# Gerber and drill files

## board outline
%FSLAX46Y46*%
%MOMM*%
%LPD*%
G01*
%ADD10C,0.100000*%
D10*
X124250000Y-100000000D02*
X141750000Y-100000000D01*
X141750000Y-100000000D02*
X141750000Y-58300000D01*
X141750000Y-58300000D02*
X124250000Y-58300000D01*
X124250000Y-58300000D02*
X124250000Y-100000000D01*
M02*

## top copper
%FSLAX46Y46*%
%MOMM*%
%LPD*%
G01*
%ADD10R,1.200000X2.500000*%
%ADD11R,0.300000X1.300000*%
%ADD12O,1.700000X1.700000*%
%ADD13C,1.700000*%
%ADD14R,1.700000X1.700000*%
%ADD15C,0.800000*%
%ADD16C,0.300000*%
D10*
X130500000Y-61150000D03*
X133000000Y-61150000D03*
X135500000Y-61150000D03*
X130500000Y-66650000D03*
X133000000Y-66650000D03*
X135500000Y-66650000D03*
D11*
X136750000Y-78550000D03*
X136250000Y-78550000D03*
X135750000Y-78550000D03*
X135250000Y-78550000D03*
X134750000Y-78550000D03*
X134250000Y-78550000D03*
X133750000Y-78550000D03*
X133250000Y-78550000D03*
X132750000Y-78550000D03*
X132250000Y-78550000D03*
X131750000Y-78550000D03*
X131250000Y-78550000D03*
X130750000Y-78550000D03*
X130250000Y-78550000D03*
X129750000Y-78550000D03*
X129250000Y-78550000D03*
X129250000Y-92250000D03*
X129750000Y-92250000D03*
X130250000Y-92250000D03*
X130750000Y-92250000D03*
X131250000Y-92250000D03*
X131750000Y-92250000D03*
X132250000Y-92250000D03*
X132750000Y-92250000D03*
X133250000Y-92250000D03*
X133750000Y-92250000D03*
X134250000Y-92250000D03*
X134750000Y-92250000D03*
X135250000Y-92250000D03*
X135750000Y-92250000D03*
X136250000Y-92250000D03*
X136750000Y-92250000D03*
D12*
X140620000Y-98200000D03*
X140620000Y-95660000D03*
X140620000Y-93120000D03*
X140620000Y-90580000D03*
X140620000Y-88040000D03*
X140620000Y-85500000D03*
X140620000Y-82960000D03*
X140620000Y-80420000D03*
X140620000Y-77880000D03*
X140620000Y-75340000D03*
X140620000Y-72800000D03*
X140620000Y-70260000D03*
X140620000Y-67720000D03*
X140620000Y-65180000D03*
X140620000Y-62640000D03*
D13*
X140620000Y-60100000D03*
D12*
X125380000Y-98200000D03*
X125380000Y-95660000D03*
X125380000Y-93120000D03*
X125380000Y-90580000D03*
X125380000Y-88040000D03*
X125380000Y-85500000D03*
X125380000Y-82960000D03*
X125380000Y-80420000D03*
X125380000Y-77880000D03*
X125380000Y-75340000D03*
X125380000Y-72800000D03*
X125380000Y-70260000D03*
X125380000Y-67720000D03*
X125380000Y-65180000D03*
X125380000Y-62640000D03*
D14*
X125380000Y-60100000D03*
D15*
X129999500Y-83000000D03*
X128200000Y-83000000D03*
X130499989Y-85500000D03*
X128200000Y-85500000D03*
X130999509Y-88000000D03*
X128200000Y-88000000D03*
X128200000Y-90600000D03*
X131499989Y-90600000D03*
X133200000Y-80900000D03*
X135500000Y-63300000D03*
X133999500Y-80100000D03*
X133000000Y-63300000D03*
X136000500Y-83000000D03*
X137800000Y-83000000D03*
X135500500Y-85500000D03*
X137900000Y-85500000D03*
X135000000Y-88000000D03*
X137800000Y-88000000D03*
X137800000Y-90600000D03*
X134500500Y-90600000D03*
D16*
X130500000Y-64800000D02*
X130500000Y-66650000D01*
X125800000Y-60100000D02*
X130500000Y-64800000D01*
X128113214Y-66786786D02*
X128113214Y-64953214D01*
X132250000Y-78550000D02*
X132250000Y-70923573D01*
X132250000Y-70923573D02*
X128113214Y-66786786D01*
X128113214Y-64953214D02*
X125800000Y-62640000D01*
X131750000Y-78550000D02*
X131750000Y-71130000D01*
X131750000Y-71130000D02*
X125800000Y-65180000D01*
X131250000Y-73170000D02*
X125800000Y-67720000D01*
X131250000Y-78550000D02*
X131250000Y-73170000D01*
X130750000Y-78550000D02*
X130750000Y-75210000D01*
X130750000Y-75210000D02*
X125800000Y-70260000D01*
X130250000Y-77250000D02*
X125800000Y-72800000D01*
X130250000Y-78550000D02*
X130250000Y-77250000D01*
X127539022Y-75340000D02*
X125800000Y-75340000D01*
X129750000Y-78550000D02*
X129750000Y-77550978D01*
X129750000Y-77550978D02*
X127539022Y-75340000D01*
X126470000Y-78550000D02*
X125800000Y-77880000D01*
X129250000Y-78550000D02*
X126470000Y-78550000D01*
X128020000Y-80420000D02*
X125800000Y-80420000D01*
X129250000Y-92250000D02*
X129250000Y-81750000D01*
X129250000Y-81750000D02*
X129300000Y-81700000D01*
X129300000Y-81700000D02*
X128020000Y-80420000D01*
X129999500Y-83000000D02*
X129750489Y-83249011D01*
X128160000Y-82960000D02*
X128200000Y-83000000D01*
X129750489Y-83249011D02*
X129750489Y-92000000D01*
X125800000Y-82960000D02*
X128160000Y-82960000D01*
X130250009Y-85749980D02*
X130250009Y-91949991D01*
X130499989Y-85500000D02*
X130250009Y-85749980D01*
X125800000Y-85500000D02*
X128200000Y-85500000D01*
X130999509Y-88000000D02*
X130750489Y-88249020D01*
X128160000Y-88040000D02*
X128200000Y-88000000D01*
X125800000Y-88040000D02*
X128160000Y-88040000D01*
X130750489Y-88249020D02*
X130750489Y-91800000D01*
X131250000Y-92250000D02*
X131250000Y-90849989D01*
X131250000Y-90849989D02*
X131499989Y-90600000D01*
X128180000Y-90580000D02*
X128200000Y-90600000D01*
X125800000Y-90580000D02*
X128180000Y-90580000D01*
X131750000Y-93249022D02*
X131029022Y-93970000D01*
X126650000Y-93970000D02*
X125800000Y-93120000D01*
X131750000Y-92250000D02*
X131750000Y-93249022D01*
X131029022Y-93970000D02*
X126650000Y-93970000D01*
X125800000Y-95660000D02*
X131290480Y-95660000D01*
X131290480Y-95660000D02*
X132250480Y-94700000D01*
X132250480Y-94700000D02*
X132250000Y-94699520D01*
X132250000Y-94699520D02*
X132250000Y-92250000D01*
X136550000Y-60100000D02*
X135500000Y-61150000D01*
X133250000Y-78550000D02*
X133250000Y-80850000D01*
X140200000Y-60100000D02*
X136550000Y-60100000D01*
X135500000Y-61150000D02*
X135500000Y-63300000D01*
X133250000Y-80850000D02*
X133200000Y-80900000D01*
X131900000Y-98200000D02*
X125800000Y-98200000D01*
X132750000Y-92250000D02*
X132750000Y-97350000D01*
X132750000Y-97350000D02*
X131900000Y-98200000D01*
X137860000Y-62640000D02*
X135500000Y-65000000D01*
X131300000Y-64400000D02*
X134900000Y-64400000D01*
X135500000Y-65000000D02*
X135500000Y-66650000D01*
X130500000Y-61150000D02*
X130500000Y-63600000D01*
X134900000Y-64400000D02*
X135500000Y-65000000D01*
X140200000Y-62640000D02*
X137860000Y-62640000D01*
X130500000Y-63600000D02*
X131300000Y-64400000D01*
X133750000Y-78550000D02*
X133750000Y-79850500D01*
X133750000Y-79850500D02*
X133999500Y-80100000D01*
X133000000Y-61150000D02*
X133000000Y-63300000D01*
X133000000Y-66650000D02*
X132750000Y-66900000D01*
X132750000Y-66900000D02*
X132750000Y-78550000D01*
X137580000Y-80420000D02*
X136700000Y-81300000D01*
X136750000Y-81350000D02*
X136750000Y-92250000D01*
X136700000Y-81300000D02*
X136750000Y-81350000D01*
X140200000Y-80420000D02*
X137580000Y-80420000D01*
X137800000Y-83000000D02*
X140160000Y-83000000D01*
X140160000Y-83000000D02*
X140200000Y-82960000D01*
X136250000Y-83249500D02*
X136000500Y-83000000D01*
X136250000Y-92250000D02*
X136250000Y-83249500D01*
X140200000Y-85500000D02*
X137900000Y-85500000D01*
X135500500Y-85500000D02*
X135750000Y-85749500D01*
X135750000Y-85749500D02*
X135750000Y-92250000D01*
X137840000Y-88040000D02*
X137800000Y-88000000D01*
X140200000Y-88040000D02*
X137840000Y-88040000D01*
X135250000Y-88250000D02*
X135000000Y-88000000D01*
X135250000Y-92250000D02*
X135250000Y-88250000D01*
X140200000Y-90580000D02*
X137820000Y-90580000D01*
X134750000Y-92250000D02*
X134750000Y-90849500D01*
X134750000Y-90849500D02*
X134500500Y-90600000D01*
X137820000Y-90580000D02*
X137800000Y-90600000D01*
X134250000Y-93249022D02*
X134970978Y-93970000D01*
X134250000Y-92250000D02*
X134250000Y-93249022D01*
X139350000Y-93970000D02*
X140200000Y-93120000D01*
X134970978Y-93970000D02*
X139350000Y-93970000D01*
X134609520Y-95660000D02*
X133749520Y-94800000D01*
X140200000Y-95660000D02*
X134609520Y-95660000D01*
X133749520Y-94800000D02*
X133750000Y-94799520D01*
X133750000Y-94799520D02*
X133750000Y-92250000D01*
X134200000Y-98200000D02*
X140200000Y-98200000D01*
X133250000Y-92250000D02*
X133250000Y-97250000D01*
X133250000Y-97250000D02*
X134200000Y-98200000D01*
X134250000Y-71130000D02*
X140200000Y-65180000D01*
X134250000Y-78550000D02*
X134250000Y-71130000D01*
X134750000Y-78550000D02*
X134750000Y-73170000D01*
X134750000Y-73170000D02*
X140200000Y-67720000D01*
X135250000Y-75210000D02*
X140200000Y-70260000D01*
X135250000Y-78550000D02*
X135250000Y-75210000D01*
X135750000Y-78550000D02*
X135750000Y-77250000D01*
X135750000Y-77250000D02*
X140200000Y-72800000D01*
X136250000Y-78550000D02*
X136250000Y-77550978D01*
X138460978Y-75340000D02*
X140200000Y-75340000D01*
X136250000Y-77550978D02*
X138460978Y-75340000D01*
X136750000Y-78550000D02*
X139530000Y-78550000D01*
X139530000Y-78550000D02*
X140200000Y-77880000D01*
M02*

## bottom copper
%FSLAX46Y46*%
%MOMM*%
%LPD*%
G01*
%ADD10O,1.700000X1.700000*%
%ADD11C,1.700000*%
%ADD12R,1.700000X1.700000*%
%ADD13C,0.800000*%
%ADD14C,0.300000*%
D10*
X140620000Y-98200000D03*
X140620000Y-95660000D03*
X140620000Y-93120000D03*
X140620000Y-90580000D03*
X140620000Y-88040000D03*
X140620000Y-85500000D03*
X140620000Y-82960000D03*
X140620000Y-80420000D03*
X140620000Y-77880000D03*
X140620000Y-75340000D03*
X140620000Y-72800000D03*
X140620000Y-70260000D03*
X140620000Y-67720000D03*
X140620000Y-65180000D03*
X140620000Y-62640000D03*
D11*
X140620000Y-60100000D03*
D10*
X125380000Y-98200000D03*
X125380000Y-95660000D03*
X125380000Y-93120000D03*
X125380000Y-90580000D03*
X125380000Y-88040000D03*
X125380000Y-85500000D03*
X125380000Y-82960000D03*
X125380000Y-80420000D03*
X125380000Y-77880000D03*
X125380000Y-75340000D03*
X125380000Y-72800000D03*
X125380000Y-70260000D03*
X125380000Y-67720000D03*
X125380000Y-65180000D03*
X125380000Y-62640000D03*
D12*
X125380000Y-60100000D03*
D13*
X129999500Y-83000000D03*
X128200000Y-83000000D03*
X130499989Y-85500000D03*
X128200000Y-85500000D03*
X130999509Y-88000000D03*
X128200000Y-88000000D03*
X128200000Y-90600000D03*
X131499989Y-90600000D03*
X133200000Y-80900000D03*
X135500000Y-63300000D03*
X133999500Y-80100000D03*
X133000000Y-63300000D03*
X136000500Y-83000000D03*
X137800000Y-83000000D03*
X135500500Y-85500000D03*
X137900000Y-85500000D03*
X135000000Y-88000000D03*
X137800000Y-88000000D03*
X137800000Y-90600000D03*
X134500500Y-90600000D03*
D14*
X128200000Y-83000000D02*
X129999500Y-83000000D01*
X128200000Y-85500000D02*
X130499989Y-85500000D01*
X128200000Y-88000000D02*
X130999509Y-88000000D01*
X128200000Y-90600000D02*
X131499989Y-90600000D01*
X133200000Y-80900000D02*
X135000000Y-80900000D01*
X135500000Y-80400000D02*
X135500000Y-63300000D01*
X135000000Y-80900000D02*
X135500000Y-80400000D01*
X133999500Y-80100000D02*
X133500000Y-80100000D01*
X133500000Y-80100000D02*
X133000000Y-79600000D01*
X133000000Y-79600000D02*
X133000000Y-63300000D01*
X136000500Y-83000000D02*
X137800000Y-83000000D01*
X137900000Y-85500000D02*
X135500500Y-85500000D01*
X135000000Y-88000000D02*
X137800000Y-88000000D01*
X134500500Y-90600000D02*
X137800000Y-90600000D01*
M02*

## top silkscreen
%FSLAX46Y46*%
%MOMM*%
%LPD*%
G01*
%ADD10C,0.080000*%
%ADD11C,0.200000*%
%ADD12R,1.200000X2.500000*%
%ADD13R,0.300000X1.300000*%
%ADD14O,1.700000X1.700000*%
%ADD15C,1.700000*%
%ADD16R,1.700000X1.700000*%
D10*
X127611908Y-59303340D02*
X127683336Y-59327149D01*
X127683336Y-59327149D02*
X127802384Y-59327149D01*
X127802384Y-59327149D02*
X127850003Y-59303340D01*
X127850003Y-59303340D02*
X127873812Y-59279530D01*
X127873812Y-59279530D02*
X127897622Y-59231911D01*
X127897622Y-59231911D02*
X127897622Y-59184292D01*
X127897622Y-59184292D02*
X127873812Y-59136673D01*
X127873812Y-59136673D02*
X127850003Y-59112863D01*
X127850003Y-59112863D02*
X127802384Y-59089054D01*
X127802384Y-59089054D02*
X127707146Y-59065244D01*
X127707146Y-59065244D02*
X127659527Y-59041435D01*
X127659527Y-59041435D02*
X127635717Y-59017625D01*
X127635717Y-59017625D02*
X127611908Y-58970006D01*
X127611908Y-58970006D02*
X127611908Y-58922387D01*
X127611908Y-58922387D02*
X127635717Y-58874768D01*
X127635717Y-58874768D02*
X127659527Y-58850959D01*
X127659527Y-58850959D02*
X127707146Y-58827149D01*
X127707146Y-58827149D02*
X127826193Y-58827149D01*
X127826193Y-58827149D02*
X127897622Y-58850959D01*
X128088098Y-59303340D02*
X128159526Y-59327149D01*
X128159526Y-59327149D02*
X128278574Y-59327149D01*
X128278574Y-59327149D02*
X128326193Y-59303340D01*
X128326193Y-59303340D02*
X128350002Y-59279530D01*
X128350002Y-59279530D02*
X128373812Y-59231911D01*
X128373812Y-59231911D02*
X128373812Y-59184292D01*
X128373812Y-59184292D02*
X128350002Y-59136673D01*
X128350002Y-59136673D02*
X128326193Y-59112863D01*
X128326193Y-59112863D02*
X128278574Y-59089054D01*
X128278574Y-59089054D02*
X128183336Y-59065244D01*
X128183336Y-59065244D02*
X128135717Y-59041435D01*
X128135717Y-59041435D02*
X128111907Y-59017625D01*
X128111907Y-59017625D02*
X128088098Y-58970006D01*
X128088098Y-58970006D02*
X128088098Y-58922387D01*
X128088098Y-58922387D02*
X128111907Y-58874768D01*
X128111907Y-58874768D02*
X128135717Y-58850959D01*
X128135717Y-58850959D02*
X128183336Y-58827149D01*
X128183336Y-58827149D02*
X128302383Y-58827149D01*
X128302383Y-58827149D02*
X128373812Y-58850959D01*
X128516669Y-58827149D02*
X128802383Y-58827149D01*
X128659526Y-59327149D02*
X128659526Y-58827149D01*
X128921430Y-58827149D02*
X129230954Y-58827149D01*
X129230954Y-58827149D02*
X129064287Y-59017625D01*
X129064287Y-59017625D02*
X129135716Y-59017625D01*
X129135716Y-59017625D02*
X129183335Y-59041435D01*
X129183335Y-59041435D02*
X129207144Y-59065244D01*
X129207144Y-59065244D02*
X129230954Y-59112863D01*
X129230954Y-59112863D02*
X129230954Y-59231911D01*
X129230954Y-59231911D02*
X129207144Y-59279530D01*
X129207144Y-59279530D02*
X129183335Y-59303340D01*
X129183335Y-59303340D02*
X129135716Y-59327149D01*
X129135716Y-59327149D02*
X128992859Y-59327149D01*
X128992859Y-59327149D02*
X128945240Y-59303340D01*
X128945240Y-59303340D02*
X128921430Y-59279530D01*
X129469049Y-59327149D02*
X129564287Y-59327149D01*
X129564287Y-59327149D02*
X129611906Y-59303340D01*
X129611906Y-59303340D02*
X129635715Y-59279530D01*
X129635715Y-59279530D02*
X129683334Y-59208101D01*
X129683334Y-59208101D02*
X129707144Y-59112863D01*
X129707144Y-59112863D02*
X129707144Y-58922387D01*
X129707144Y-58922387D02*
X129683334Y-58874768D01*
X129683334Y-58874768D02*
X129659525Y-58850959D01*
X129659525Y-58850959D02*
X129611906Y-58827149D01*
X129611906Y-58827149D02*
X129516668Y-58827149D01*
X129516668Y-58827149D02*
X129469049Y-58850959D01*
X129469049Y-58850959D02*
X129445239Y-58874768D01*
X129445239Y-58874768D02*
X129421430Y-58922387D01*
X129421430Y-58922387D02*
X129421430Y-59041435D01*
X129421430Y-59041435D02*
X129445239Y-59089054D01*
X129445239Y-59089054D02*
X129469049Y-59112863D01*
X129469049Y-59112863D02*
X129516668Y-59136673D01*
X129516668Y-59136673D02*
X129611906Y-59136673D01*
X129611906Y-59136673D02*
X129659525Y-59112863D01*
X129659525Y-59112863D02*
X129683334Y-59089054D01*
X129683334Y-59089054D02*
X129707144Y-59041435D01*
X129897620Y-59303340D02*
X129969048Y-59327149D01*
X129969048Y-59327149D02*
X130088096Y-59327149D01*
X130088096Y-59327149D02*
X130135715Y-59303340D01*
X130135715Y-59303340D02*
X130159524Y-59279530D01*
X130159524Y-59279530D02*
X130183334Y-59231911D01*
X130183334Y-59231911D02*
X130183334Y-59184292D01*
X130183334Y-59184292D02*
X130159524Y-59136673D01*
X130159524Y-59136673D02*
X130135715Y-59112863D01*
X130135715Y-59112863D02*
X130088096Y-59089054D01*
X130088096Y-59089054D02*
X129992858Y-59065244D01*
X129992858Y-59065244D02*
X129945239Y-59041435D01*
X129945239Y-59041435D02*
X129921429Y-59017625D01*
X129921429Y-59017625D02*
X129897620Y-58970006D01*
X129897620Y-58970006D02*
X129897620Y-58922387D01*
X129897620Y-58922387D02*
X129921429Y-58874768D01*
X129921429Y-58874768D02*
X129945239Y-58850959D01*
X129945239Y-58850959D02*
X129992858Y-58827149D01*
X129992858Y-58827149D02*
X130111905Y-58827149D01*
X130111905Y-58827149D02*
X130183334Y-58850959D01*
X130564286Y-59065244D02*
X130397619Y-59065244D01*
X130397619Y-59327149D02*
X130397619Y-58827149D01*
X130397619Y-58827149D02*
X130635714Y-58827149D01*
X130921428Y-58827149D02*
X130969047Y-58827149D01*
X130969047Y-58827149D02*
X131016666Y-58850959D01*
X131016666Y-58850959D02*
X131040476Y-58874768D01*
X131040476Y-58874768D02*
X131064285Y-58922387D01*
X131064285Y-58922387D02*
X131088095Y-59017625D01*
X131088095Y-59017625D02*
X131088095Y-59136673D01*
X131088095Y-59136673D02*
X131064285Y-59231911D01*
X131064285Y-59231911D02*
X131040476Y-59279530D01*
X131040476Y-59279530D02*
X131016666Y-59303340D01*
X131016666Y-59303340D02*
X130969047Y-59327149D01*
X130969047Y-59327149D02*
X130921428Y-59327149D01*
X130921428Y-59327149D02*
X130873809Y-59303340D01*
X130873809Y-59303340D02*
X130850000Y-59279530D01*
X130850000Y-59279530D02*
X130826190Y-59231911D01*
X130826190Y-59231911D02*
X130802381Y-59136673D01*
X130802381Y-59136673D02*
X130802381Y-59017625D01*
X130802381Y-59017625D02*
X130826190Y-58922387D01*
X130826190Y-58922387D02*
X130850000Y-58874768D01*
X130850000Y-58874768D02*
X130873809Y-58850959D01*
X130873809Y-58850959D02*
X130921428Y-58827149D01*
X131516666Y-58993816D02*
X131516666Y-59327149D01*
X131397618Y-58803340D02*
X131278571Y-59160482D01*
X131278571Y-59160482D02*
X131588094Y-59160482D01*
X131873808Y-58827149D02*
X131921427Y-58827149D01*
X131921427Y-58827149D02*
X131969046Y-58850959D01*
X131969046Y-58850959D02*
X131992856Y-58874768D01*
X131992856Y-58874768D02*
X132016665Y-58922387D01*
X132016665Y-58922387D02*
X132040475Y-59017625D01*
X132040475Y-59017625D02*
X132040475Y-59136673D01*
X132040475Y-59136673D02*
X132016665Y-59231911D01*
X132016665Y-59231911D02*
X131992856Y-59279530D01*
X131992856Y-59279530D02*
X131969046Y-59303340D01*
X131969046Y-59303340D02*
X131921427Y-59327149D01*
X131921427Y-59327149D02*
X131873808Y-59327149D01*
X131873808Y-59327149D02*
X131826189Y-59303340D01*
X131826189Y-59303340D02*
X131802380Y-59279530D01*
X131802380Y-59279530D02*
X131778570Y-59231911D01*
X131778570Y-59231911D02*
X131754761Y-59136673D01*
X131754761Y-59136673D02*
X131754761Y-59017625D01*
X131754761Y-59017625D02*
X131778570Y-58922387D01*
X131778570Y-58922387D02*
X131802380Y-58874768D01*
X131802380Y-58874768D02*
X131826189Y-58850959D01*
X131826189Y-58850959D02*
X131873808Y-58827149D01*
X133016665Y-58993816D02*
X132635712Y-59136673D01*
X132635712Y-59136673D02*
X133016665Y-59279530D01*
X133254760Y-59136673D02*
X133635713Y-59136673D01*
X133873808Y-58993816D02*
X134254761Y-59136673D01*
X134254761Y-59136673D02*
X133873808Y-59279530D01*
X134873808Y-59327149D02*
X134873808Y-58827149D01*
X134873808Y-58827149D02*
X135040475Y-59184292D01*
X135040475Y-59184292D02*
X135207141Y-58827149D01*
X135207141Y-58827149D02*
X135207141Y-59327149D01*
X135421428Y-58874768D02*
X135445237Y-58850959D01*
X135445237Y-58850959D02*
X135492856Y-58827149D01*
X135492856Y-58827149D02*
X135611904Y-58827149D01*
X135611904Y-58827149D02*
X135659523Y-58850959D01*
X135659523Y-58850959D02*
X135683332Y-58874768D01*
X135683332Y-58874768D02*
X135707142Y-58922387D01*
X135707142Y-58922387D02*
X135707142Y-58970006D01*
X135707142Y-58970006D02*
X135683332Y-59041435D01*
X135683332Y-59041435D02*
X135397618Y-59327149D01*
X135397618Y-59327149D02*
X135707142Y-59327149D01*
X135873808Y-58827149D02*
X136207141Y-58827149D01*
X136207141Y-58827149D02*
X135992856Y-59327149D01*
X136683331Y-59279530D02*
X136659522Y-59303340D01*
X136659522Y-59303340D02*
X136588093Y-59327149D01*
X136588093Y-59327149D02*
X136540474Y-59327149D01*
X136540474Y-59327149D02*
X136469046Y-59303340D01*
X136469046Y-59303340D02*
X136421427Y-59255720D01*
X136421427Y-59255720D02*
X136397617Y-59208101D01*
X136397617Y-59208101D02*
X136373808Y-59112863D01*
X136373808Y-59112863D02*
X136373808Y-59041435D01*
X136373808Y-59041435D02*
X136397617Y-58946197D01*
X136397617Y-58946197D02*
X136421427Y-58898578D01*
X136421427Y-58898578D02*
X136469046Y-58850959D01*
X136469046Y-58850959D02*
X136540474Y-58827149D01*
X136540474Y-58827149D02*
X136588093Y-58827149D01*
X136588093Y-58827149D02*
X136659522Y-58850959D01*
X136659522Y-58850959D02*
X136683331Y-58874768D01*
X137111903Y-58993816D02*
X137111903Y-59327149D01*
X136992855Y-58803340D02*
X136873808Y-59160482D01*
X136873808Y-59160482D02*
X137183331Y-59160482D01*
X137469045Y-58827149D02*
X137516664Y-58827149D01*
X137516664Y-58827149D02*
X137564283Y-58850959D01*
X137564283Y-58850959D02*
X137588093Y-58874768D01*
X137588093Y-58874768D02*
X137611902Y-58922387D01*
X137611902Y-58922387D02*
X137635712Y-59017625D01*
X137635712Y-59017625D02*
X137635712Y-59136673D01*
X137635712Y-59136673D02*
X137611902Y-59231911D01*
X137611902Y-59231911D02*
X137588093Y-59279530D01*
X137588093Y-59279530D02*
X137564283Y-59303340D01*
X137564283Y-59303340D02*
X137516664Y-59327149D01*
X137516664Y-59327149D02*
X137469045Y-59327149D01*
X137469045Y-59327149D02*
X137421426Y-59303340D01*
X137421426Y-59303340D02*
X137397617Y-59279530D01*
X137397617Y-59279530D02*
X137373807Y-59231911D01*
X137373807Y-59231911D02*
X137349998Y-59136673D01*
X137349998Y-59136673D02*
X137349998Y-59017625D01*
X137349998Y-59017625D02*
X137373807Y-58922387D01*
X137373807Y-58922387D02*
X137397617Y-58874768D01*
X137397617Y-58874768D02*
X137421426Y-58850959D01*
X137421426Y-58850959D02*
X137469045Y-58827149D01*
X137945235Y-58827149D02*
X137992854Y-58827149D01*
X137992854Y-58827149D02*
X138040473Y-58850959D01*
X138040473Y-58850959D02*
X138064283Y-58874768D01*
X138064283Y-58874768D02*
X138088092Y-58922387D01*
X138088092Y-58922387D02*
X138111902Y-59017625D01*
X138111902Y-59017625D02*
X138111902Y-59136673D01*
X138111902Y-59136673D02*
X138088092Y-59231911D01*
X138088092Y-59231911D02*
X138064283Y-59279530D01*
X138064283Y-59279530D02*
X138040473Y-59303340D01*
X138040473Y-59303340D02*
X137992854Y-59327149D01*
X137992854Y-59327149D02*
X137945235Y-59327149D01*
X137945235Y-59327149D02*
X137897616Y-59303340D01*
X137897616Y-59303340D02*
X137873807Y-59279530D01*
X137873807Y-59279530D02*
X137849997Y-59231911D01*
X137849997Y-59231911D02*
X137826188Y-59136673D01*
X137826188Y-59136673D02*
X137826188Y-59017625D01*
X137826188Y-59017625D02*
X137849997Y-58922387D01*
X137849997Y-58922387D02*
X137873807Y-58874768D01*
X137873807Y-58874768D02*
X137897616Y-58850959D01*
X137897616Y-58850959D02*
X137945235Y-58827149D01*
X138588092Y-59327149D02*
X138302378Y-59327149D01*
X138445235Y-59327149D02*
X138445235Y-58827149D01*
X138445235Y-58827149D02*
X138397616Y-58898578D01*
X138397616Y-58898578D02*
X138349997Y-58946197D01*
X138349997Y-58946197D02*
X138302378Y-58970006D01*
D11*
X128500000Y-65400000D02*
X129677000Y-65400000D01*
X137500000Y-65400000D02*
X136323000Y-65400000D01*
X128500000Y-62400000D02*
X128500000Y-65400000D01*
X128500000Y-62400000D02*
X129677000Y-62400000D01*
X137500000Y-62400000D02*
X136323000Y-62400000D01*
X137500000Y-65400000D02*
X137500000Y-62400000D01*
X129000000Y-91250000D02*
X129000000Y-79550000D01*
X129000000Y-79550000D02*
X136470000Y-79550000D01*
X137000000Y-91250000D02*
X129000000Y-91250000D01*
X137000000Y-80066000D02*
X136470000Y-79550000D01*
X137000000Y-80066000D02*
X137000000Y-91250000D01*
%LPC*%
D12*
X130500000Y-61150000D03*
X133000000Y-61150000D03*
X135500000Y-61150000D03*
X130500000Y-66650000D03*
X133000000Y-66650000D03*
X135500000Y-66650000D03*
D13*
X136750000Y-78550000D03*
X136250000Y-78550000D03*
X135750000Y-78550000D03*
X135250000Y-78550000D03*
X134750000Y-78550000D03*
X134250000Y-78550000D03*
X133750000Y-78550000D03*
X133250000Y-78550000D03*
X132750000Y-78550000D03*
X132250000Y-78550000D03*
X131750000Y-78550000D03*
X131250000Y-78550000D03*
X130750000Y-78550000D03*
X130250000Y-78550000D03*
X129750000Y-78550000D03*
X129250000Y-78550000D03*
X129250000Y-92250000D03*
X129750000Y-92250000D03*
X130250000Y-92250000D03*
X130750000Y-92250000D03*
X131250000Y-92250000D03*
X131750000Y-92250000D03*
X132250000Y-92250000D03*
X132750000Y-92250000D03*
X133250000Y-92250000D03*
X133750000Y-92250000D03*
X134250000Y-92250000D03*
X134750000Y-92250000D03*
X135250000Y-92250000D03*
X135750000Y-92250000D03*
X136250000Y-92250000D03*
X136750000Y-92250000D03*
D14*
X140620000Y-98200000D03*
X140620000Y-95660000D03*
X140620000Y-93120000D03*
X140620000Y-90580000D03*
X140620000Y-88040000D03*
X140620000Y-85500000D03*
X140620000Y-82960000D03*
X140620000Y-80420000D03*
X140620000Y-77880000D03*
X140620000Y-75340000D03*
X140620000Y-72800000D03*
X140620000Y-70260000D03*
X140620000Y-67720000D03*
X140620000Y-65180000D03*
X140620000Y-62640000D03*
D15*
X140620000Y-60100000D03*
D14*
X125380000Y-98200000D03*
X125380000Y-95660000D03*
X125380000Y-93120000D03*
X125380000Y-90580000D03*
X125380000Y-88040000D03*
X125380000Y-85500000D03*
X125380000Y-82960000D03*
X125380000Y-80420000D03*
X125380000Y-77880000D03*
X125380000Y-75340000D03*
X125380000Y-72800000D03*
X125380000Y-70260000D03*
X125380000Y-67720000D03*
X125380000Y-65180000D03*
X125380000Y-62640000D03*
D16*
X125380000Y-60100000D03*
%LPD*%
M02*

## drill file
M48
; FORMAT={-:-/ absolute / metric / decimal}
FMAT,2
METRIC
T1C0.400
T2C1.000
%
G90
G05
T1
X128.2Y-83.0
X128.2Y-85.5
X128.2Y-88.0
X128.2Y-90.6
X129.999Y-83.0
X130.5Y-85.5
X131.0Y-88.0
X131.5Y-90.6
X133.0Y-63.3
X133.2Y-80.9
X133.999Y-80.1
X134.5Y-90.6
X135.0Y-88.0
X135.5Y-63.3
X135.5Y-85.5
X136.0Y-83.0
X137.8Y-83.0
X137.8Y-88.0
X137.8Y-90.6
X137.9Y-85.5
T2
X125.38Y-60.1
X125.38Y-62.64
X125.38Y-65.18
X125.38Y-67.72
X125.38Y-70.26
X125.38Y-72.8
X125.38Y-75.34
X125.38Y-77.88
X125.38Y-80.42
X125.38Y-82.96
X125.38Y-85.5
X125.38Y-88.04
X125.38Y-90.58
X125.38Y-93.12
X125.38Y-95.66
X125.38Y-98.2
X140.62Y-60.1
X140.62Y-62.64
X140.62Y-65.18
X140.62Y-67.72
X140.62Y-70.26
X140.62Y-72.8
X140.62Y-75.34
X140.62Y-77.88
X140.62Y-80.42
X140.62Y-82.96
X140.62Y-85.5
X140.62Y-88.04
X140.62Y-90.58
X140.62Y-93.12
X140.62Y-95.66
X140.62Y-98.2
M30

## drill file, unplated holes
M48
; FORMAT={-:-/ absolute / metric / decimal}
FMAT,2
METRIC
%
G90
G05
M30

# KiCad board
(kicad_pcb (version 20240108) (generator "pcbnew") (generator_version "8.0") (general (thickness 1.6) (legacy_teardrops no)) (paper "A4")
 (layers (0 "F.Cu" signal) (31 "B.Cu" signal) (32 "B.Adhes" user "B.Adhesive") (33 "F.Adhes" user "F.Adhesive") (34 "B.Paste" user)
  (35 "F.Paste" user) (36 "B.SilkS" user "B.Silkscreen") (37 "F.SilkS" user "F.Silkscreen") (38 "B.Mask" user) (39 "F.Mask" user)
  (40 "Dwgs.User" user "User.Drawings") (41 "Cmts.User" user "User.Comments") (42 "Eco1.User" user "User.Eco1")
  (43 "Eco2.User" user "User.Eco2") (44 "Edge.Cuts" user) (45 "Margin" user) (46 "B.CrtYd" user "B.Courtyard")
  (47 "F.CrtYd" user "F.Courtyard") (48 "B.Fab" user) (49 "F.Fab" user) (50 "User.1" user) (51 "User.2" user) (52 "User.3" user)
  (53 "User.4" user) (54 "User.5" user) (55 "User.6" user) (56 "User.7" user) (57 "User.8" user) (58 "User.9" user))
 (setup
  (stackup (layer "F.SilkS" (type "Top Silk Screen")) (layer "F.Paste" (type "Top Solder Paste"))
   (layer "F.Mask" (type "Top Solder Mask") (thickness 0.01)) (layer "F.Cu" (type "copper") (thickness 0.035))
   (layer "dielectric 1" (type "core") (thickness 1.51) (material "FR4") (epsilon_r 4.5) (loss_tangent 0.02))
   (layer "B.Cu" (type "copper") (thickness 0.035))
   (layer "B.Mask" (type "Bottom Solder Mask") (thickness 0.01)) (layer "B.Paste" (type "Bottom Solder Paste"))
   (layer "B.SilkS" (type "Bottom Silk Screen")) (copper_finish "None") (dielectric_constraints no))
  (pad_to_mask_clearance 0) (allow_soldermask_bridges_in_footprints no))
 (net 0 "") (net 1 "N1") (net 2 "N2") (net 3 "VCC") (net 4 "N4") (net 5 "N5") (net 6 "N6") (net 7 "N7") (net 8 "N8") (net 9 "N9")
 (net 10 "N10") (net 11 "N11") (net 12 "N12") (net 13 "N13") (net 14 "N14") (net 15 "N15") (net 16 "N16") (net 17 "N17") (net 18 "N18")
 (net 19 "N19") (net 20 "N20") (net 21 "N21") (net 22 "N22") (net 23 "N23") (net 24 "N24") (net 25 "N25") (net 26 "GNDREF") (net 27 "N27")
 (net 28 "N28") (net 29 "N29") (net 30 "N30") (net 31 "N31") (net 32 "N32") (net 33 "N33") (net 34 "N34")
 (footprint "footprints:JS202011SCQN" (layer "F.Cu") (at 133 63.9)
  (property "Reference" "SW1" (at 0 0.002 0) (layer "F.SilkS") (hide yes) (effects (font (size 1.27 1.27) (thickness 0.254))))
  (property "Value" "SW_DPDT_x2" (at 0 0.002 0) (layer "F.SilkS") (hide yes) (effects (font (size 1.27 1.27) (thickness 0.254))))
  (fp_line (start -4.5 -1.5) (end -4.5 1.5) (stroke (width 0.2) (type solid)) (layer "F.SilkS"))
  (fp_line (start -4.5 -1.5) (end -3.323 -1.5) (stroke (width 0.2) (type solid)) (layer "F.SilkS"))
  (fp_line (start -4.5 1.5) (end -3.323 1.5) (stroke (width 0.2) (type solid)) (layer "F.SilkS"))
  (fp_line (start 4.5 -1.5) (end 3.323 -1.5) (stroke (width 0.2) (type solid)) (layer "F.SilkS"))
  (fp_line (start 4.5 1.5) (end 3.323 1.5) (stroke (width 0.2) (type solid)) (layer "F.SilkS"))
  (fp_line (start 4.5 1.5) (end 4.5 -1.5) (stroke (width 0.2) (type solid)) (layer "F.SilkS"))
  (pad "1" smd rect (at -2.5 -2.75) (size 1.2 2.5) (layers "F.Cu" "F.Paste" "F.Mask") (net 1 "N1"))
  (pad "2" smd rect (at 0 -2.75) (size 1.2 2.5) (layers "F.Cu" "F.Paste" "F.Mask") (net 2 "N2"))
  (pad "3" smd rect (at 2.5 -2.75) (size 1.2 2.5) (layers "F.Cu" "F.Paste" "F.Mask") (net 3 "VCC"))
  (pad "4" smd rect (at -2.5 2.75) (size 1.2 2.5) (layers "F.Cu" "F.Paste" "F.Mask") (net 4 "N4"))
  (pad "5" smd rect (at 0 2.75) (size 1.2 2.5) (layers "F.Cu" "F.Paste" "F.Mask") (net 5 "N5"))
  (pad "6" smd rect (at 2.5 2.75) (size 1.2 2.5) (layers "F.Cu" "F.Paste" "F.Mask") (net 1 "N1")))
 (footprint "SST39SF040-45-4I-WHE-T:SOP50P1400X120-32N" (layer "F.Cu") (at 133 85.4 -90)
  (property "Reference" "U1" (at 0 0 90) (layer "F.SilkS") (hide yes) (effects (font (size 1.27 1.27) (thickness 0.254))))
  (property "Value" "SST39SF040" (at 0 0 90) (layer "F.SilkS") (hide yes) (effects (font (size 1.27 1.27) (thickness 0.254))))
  (fp_line (start -5.85 4) (end -5.85 -3.47) (stroke (width 0.2) (type solid)) (layer "F.SilkS"))
  (fp_line (start 5.85 4) (end -5.85 4) (stroke (width 0.2) (type solid)) (layer "F.SilkS"))
  (fp_line (start -5.334 -4) (end -5.85 -3.47) (stroke (width 0.2) (type solid)) (layer "F.SilkS"))
  (fp_line (start -5.334 -4) (end 5.85 -4) (stroke (width 0.2) (type solid)) (layer "F.SilkS"))
  (fp_line (start 5.85 -4) (end 5.85 4) (stroke (width 0.2) (type solid)) (layer "F.SilkS"))
  (pad "1" smd rect (at -6.85 -3.75) (size 0.3 1.3) (layers "F.Cu" "F.Paste" "F.Mask") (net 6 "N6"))
  (pad "2" smd rect (at -6.85 -3.25) (size 0.3 1.3) (layers "F.Cu" "F.Paste" "F.Mask") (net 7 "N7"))
  (pad "3" smd rect (at -6.85 -2.75) (size 0.3 1.3) (layers "F.Cu" "F.Paste" "F.Mask") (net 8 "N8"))
  (pad "4" smd rect (at -6.85 -2.25) (size 0.3 1.3) (layers "F.Cu" "F.Paste" "F.Mask") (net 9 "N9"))
  (pad "5" smd rect (at -6.85 -1.75) (size 0.3 1.3) (layers "F.Cu" "F.Paste" "F.Mask") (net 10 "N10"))
  (pad "6" smd rect (at -6.85 -1.25) (size 0.3 1.3) (layers "F.Cu" "F.Paste" "F.Mask") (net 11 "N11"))
  (pad "7" smd rect (at -6.85 -0.75) (size 0.3 1.3) (layers "F.Cu" "F.Paste" "F.Mask") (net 2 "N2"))
  (pad "8" smd rect (at -6.85 -0.25) (size 0.3 1.3) (layers "F.Cu" "F.Paste" "F.Mask") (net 3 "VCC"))
  (pad "9" smd rect (at -6.85 0.25) (size 0.3 1.3) (layers "F.Cu" "F.Paste" "F.Mask") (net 5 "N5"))
  (pad "10" smd rect (at -6.85 0.75) (size 0.3 1.3) (layers "F.Cu" "F.Paste" "F.Mask") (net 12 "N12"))
  (pad "11" smd rect (at -6.85 1.25) (size 0.3 1.3) (layers "F.Cu" "F.Paste" "F.Mask") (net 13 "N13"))
  (pad "12" smd rect (at -6.85 1.75) (size 0.3 1.3) (layers "F.Cu" "F.Paste" "F.Mask") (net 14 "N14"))
  (pad "13" smd rect (at -6.85 2.25) (size 0.3 1.3) (layers "F.Cu" "F.Paste" "F.Mask") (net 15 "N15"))
  (pad "14" smd rect (at -6.85 2.75) (size 0.3 1.3) (layers "F.Cu" "F.Paste" "F.Mask") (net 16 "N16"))
  (pad "15" smd rect (at -6.85 3.25) (size 0.3 1.3) (layers "F.Cu" "F.Paste" "F.Mask") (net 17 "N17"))
  (pad "16" smd rect (at -6.85 3.75) (size 0.3 1.3) (layers "F.Cu" "F.Paste" "F.Mask") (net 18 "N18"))
  (pad "17" smd rect (at 6.85 3.75) (size 0.3 1.3) (layers "F.Cu" "F.Paste" "F.Mask") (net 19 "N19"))
  (pad "18" smd rect (at 6.85 3.25) (size 0.3 1.3) (layers "F.Cu" "F.Paste" "F.Mask") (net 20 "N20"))
  (pad "19" smd rect (at 6.85 2.75) (size 0.3 1.3) (layers "F.Cu" "F.Paste" "F.Mask") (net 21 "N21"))
  (pad "20" smd rect (at 6.85 2.25) (size 0.3 1.3) (layers "F.Cu" "F.Paste" "F.Mask") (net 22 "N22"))
  (pad "21" smd rect (at 6.85 1.75) (size 0.3 1.3) (layers "F.Cu" "F.Paste" "F.Mask") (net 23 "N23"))
  (pad "22" smd rect (at 6.85 1.25) (size 0.3 1.3) (layers "F.Cu" "F.Paste" "F.Mask") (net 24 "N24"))
  (pad "23" smd rect (at 6.85 0.75) (size 0.3 1.3) (layers "F.Cu" "F.Paste" "F.Mask") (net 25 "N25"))
  (pad "24" smd rect (at 6.85 0.25) (size 0.3 1.3) (layers "F.Cu" "F.Paste" "F.Mask") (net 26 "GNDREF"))
  (pad "25" smd rect (at 6.85 -0.25) (size 0.3 1.3) (layers "F.Cu" "F.Paste" "F.Mask") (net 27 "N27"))
  (pad "26" smd rect (at 6.85 -0.75) (size 0.3 1.3) (layers "F.Cu" "F.Paste" "F.Mask") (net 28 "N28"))
  (pad "27" smd rect (at 6.85 -1.25) (size 0.3 1.3) (layers "F.Cu" "F.Paste" "F.Mask") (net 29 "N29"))
  (pad "28" smd rect (at 6.85 -1.75) (size 0.3 1.3) (layers "F.Cu" "F.Paste" "F.Mask") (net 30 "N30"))
  (pad "29" smd rect (at 6.85 -2.25) (size 0.3 1.3) (layers "F.Cu" "F.Paste" "F.Mask") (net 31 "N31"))
  (pad "30" smd rect (at 6.85 -2.75) (size 0.3 1.3) (layers "F.Cu" "F.Paste" "F.Mask") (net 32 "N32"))
  (pad "31" smd rect (at 6.85 -3.25) (size 0.3 1.3) (layers "F.Cu" "F.Paste" "F.Mask") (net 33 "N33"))
  (pad "32" smd rect (at 6.85 -3.75) (size 0.3 1.3) (layers "F.Cu" "F.Paste" "F.Mask") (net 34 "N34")))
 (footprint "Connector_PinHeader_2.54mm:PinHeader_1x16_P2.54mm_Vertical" (layer "F.Cu") (at 140.62 60.1)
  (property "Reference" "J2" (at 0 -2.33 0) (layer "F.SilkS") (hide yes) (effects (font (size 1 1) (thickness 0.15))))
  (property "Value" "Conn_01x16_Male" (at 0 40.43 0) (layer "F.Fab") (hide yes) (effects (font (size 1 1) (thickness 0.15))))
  (pad "17" thru_hole oval (at 0 38.1) (size 1.7 1.7) (drill 1) (layers "*.Cu" "*.Mask") (remove_unused_layers no) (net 27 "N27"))
  (pad "18" thru_hole oval (at 0 35.56) (size 1.7 1.7) (drill 1) (layers "*.Cu" "*.Mask") (remove_unused_layers no) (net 28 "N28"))
  (pad "19" thru_hole oval (at 0 33.02) (size 1.7 1.7) (drill 1) (layers "*.Cu" "*.Mask") (remove_unused_layers no) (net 29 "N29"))
  (pad "20" thru_hole oval (at 0 30.48) (size 1.7 1.7) (drill 1) (layers "*.Cu" "*.Mask") (remove_unused_layers no) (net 30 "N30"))
  (pad "21" thru_hole oval (at 0 27.94) (size 1.7 1.7) (drill 1) (layers "*.Cu" "*.Mask") (remove_unused_layers no) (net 31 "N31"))
  (pad "22" thru_hole oval (at 0 25.4) (size 1.7 1.7) (drill 1) (layers "*.Cu" "*.Mask") (remove_unused_layers no) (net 32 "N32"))
  (pad "23" thru_hole oval (at 0 22.86) (size 1.7 1.7) (drill 1) (layers "*.Cu" "*.Mask") (remove_unused_layers no) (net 33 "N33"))
  (pad "24" thru_hole oval (at 0 20.32) (size 1.7 1.7) (drill 1) (layers "*.Cu" "*.Mask") (remove_unused_layers no) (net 34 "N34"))
  (pad "25" thru_hole oval (at 0 17.78) (size 1.7 1.7) (drill 1) (layers "*.Cu" "*.Mask") (remove_unused_layers no) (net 6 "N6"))
  (pad "26" thru_hole oval (at 0 15.24) (size 1.7 1.7) (drill 1) (layers "*.Cu" "*.Mask") (remove_unused_layers no) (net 7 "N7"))
  (pad "27" thru_hole oval (at 0 12.7) (size 1.7 1.7) (drill 1) (layers "*.Cu" "*.Mask") (remove_unused_layers no) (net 8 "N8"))
  (pad "28" thru_hole oval (at 0 10.16) (size 1.7 1.7) (drill 1) (layers "*.Cu" "*.Mask") (remove_unused_layers no) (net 9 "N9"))
  (pad "29" thru_hole oval (at 0 7.62) (size 1.7 1.7) (drill 1) (layers "*.Cu" "*.Mask") (remove_unused_layers no) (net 10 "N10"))
  (pad "30" thru_hole oval (at 0 5.08) (size 1.7 1.7) (drill 1) (layers "*.Cu" "*.Mask") (remove_unused_layers no) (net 11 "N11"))
  (pad "31" thru_hole oval (at 0 2.54) (size 1.7 1.7) (drill 1) (layers "*.Cu" "*.Mask") (remove_unused_layers no) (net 1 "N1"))
  (pad "32" thru_hole circle (at 0 0) (size 1.7 1.7) (drill 1) (layers "*.Cu" "*.Mask") (remove_unused_layers no) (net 3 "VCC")))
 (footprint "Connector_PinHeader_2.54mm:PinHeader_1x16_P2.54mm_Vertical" (layer "F.Cu") (at 125.38 60.1)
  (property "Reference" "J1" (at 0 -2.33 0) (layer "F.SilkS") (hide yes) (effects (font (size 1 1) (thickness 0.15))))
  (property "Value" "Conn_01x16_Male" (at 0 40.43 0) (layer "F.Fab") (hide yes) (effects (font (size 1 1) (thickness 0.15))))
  (pad "1" thru_hole rect (at 0 0) (size 1.7 1.7) (drill 1) (layers "*.Cu" "*.Mask") (remove_unused_layers no) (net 4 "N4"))
  (pad "2" thru_hole oval (at 0 2.54) (size 1.7 1.7) (drill 1) (layers "*.Cu" "*.Mask") (remove_unused_layers no) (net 12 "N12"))
  (pad "3" thru_hole oval (at 0 5.08) (size 1.7 1.7) (drill 1) (layers "*.Cu" "*.Mask") (remove_unused_layers no) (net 13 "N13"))
  (pad "4" thru_hole oval (at 0 7.62) (size 1.7 1.7) (drill 1) (layers "*.Cu" "*.Mask") (remove_unused_layers no) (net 14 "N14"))
  (pad "5" thru_hole oval (at 0 10.16) (size 1.7 1.7) (drill 1) (layers "*.Cu" "*.Mask") (remove_unused_layers no) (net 15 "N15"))
  (pad "6" thru_hole oval (at 0 12.7) (size 1.7 1.7) (drill 1) (layers "*.Cu" "*.Mask") (remove_unused_layers no) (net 16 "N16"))
  (pad "7" thru_hole oval (at 0 15.24) (size 1.7 1.7) (drill 1) (layers "*.Cu" "*.Mask") (remove_unused_layers no) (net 17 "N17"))
  (pad "8" thru_hole oval (at 0 17.78) (size 1.7 1.7) (drill 1) (layers "*.Cu" "*.Mask") (remove_unused_layers no) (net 18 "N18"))
  (pad "9" thru_hole oval (at 0 20.32) (size 1.7 1.7) (drill 1) (layers "*.Cu" "*.Mask") (remove_unused_layers no) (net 19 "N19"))
  (pad "10" thru_hole oval (at 0 22.86) (size 1.7 1.7) (drill 1) (layers "*.Cu" "*.Mask") (remove_unused_layers no) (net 20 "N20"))
  (pad "11" thru_hole oval (at 0 25.4) (size 1.7 1.7) (drill 1) (layers "*.Cu" "*.Mask") (remove_unused_layers no) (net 21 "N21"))
  (pad "12" thru_hole oval (at 0 27.94) (size 1.7 1.7) (drill 1) (layers "*.Cu" "*.Mask") (remove_unused_layers no) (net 22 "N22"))
  (pad "13" thru_hole oval (at 0 30.48) (size 1.7 1.7) (drill 1) (layers "*.Cu" "*.Mask") (remove_unused_layers no) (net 23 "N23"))
  (pad "14" thru_hole oval (at 0 33.02) (size 1.7 1.7) (drill 1) (layers "*.Cu" "*.Mask") (remove_unused_layers no) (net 24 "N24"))
  (pad "15" thru_hole oval (at 0 35.56) (size 1.7 1.7) (drill 1) (layers "*.Cu" "*.Mask") (remove_unused_layers no) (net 25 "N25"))
  (pad "16" thru_hole oval (at 0 38.1) (size 1.7 1.7) (drill 1) (layers "*.Cu" "*.Mask") (remove_unused_layers no) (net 26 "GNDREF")))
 (gr_line (start 124.25 100) (end 141.75 100) (stroke (width 0.1) (type solid)) (layer "Edge.Cuts"))
 (gr_line (start 141.75 100) (end 141.75 58.3) (stroke (width 0.1) (type solid)) (layer "Edge.Cuts"))
 (gr_line (start 141.75 58.3) (end 124.25 58.3) (stroke (width 0.1) (type solid)) (layer "Edge.Cuts"))
 (gr_line (start 124.25 58.3) (end 124.25 100) (stroke (width 0.1) (type solid)) (layer "Edge.Cuts"))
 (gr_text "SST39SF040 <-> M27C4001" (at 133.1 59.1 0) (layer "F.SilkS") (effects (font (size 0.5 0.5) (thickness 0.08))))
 (segment (start 130.5 64.8) (end 130.5 66.65) (width 0.3) (layer "F.Cu") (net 4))
 (segment (start 125.8 60.1) (end 130.5 64.8) (width 0.3) (layer "F.Cu") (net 4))
 (segment (start 128.113214 66.786786) (end 128.113214 64.953214) (width 0.3) (layer "F.Cu") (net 12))
 (segment (start 132.25 78.55) (end 132.25 70.923573) (width 0.3) (layer "F.Cu") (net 12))
 (segment (start 132.25 70.923573) (end 128.113214 66.786786) (width 0.3) (layer "F.Cu") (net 12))
 (segment (start 128.113214 64.953214) (end 125.8 62.64) (width 0.3) (layer "F.Cu") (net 12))
 (segment (start 131.75 78.55) (end 131.75 71.13) (width 0.3) (layer "F.Cu") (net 13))
 (segment (start 131.75 71.13) (end 125.8 65.18) (width 0.3) (layer "F.Cu") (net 13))
 (segment (start 131.25 73.17) (end 125.8 67.72) (width 0.3) (layer "F.Cu") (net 14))
 (segment (start 131.25 78.55) (end 131.25 73.17) (width 0.3) (layer "F.Cu") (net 14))
 (segment (start 130.75 78.55) (end 130.75 75.21) (width 0.3) (layer "F.Cu") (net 15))
 (segment (start 130.75 75.21) (end 125.8 70.26) (width 0.3) (layer "F.Cu") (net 15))
 (segment (start 130.25 77.25) (end 125.8 72.8) (width 0.3) (layer "F.Cu") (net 16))
 (segment (start 130.25 78.55) (end 130.25 77.25) (width 0.3) (layer "F.Cu") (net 16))
 (segment (start 127.539022 75.34) (end 125.8 75.34) (width 0.3) (layer "F.Cu") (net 17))
 (segment (start 129.75 78.55) (end 129.75 77.550978) (width 0.3) (layer "F.Cu") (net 17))
 (segment (start 129.75 77.550978) (end 127.539022 75.34) (width 0.3) (layer "F.Cu") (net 17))
 (segment (start 126.47 78.55) (end 125.8 77.88) (width 0.3) (layer "F.Cu") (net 18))
 (segment (start 129.25 78.55) (end 126.47 78.55) (width 0.3) (layer "F.Cu") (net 18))
 (segment (start 128.02 80.42) (end 125.8 80.42) (width 0.3) (layer "F.Cu") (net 19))
 (segment (start 129.25 92.25) (end 129.25 81.75) (width 0.3) (layer "F.Cu") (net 19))
 (segment (start 129.25 81.75) (end 129.3 81.7) (width 0.3) (layer "F.Cu") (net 19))
 (segment (start 129.3 81.7) (end 128.02 80.42) (width 0.3) (layer "F.Cu") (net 19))
 (segment (start 129.9995 83) (end 129.750489 83.249011) (width 0.3) (layer "F.Cu") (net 20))
 (segment (start 128.16 82.96) (end 128.2 83) (width 0.3) (layer "F.Cu") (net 20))
 (segment (start 129.750489 83.249011) (end 129.750489 92) (width 0.3) (layer "F.Cu") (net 20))
 (segment (start 125.8 82.96) (end 128.16 82.96) (width 0.3) (layer "F.Cu") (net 20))
 (via (at 129.9995 83) (size 0.8) (drill 0.4) (layers "F.Cu" "B.Cu") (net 20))
 (via (at 128.2 83) (size 0.8) (drill 0.4) (layers "F.Cu" "B.Cu") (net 20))
 (segment (start 128.2 83) (end 129.9995 83) (width 0.3) (layer "B.Cu") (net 20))
 (segment (start 130.250009 85.74998) (end 130.250009 91.949991) (width 0.3) (layer "F.Cu") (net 21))
 (segment (start 130.499989 85.5) (end 130.250009 85.74998) (width 0.3) (layer "F.Cu") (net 21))
 (segment (start 125.8 85.5) (end 128.2 85.5) (width 0.3) (layer "F.Cu") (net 21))
 (via (at 130.499989 85.5) (size 0.8) (drill 0.4) (layers "F.Cu" "B.Cu") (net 21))
 (via (at 128.2 85.5) (size 0.8) (drill 0.4) (layers "F.Cu" "B.Cu") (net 21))
 (segment (start 128.2 85.5) (end 130.499989 85.5) (width 0.3) (layer "B.Cu") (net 21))
 (segment (start 130.999509 88) (end 130.750489 88.24902) (width 0.3) (layer "F.Cu") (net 22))
 (segment (start 128.16 88.04) (end 128.2 88) (width 0.3) (layer "F.Cu") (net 22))
 (segment (start 125.8 88.04) (end 128.16 88.04) (width 0.3) (layer "F.Cu") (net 22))
 (segment (start 130.750489 88.24902) (end 130.750489 91.8) (width 0.3) (layer "F.Cu") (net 22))
 (via (at 130.999509 88) (size 0.8) (drill 0.4) (layers "F.Cu" "B.Cu") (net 22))
 (via (at 128.2 88) (size 0.8) (drill 0.4) (layers "F.Cu" "B.Cu") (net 22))
 (segment (start 128.2 88) (end 130.999509 88) (width 0.3) (layer "B.Cu") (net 22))
 (segment (start 131.25 92.25) (end 131.25 90.849989) (width 0.3) (layer "F.Cu") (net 23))
 (segment (start 131.25 90.849989) (end 131.499989 90.6) (width 0.3) (layer "F.Cu") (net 23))
 (segment (start 128.18 90.58) (end 128.2 90.6) (width 0.3) (layer "F.Cu") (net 23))
 (segment (start 125.8 90.58) (end 128.18 90.58) (width 0.3) (layer "F.Cu") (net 23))
 (via (at 128.2 90.6) (size 0.8) (drill 0.4) (layers "F.Cu" "B.Cu") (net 23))
 (via (at 131.499989 90.6) (size 0.8) (drill 0.4) (layers "F.Cu" "B.Cu") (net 23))
 (segment (start 128.2 90.6) (end 131.499989 90.6) (width 0.3) (layer "B.Cu") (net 23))
 (segment (start 131.75 93.249022) (end 131.029022 93.97) (width 0.3) (layer "F.Cu") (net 24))
 (segment (start 126.65 93.97) (end 125.8 93.12) (width 0.3) (layer "F.Cu") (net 24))
 (segment (start 131.75 92.25) (end 131.75 93.249022) (width 0.3) (layer "F.Cu") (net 24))
 (segment (start 131.029022 93.97) (end 126.65 93.97) (width 0.3) (layer "F.Cu") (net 24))
 (segment (start 125.8 95.66) (end 131.29048 95.66) (width 0.3) (layer "F.Cu") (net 25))
 (segment (start 131.29048 95.66) (end 132.25048 94.7) (width 0.3) (layer "F.Cu") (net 25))
 (segment (start 132.25048 94.7) (end 132.25 94.69952) (width 0.3) (layer "F.Cu") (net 25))
 (segment (start 132.25 94.69952) (end 132.25 92.25) (width 0.3) (layer "F.Cu") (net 25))
 (segment (start 136.55 60.1) (end 135.5 61.15) (width 0.3) (layer "F.Cu") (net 3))
 (segment (start 133.25 78.55) (end 133.25 80.85) (width 0.3) (layer "F.Cu") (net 3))
 (segment (start 140.2 60.1) (end 136.55 60.1) (width 0.3) (layer "F.Cu") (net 3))
 (segment (start 135.5 61.15) (end 135.5 63.3) (width 0.3) (layer "F.Cu") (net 3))
 (segment (start 133.25 80.85) (end 133.2 80.9) (width 0.3) (layer "F.Cu") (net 3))
 (via (at 133.2 80.9) (size 0.8) (drill 0.4) (layers "F.Cu" "B.Cu") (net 3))
 (via (at 135.5 63.3) (size 0.8) (drill 0.4) (layers "F.Cu" "B.Cu") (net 3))
 (segment (start 133.2 80.9) (end 135 80.9) (width 0.3) (layer "B.Cu") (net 3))
 (segment (start 135.5 80.4) (end 135.5 63.3) (width 0.3) (layer "B.Cu") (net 3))
 (segment (start 135 80.9) (end 135.5 80.4) (width 0.3) (layer "B.Cu") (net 3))
 (segment (start 131.9 98.2) (end 125.8 98.2) (width 0.3) (layer "F.Cu") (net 26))
 (segment (start 132.75 92.25) (end 132.75 97.35) (width 0.3) (layer "F.Cu") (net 26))
 (segment (start 132.75 97.35) (end 131.9 98.2) (width 0.3) (layer "F.Cu") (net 26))
 (segment (start 137.86 62.64) (end 135.5 65) (width 0.3) (layer "F.Cu") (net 1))
 (segment (start 131.3 64.4) (end 134.9 64.4) (width 0.3) (layer "F.Cu") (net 1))
 (segment (start 135.5 65) (end 135.5 66.65) (width 0.3) (layer "F.Cu") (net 1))
 (segment (start 130.5 61.15) (end 130.5 63.6) (width 0.3) (layer "F.Cu") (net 1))
 (segment (start 134.9 64.4) (end 135.5 65) (width 0.3) (layer "F.Cu") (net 1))
 (segment (start 140.2 62.64) (end 137.86 62.64) (width 0.3) (layer "F.Cu") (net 1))
 (segment (start 130.5 63.6) (end 131.3 64.4) (width 0.3) (layer "F.Cu") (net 1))
 (segment (start 133.75 78.55) (end 133.75 79.8505) (width 0.3) (layer "F.Cu") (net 2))
 (segment (start 133.75 79.8505) (end 133.9995 80.1) (width 0.3) (layer "F.Cu") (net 2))
 (segment (start 133 61.15) (end 133 63.3) (width 0.3) (layer "F.Cu") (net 2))
 (via (at 133.9995 80.1) (size 0.8) (drill 0.4) (layers "F.Cu" "B.Cu") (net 2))
 (via (at 133 63.3) (size 0.8) (drill 0.4) (layers "F.Cu" "B.Cu") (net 2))
 (segment (start 133.9995 80.1) (end 133.5 80.1) (width 0.3) (layer "B.Cu") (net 2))
 (segment (start 133.5 80.1) (end 133 79.6) (width 0.3) (layer "B.Cu") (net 2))
 (segment (start 133 79.6) (end 133 63.3) (width 0.3) (layer "B.Cu") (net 2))
 (segment (start 133 66.65) (end 132.75 66.9) (width 0.3) (layer "F.Cu") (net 5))
 (segment (start 132.75 66.9) (end 132.75 78.55) (width 0.3) (layer "F.Cu") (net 5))
 (segment (start 137.58 80.42) (end 136.7 81.3) (width 0.3) (layer "F.Cu") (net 34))
 (segment (start 136.75 81.35) (end 136.75 92.25) (width 0.3) (layer "F.Cu") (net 34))
 (segment (start 136.7 81.3) (end 136.75 81.35) (width 0.3) (layer "F.Cu") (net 34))
 (segment (start 140.2 80.42) (end 137.58 80.42) (width 0.3) (layer "F.Cu") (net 34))
 (segment (start 137.8 83) (end 140.16 83) (width 0.3) (layer "F.Cu") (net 33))
 (segment (start 140.16 83) (end 140.2 82.96) (width 0.3) (layer "F.Cu") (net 33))
 (segment (start 136.25 83.2495) (end 136.0005 83) (width 0.3) (layer "F.Cu") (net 33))
 (segment (start 136.25 92.25) (end 136.25 83.2495) (width 0.3) (layer "F.Cu") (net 33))
 (via (at 136.0005 83) (size 0.8) (drill 0.4) (layers "F.Cu" "B.Cu") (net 33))
 (via (at 137.8 83) (size 0.8) (drill 0.4) (layers "F.Cu" "B.Cu") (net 33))
 (segment (start 136.0005 83) (end 137.8 83) (width 0.3) (layer "B.Cu") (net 33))
 (segment (start 140.2 85.5) (end 137.9 85.5) (width 0.3) (layer "F.Cu") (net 32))
 (segment (start 135.5005 85.5) (end 135.75 85.7495) (width 0.3) (layer "F.Cu") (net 32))
 (segment (start 135.75 85.7495) (end 135.75 92.25) (width 0.3) (layer "F.Cu") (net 32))
 (via (at 135.5005 85.5) (size 0.8) (drill 0.4) (layers "F.Cu" "B.Cu") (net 32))
 (via (at 137.9 85.5) (size 0.8) (drill 0.4) (layers "F.Cu" "B.Cu") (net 32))
 (segment (start 137.9 85.5) (end 135.5005 85.5) (width 0.3) (layer "B.Cu") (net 32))
 (segment (start 137.84 88.04) (end 137.8 88) (width 0.3) (layer "F.Cu") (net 31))
 (segment (start 140.2 88.04) (end 137.84 88.04) (width 0.3) (layer "F.Cu") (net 31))
 (segment (start 135.25 88.25) (end 135 88) (width 0.3) (layer "F.Cu") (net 31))
 (segment (start 135.25 92.25) (end 135.25 88.25) (width 0.3) (layer "F.Cu") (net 31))
 (via (at 135 88) (size 0.8) (drill 0.4) (layers "F.Cu" "B.Cu") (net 31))
 (via (at 137.8 88) (size 0.8) (drill 0.4) (layers "F.Cu" "B.Cu") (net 31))
 (segment (start 135 88) (end 137.8 88) (width 0.3) (layer "B.Cu") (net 31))
 (segment (start 140.2 90.58) (end 137.82 90.58) (width 0.3) (layer "F.Cu") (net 30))
 (segment (start 134.75 92.25) (end 134.75 90.8495) (width 0.3) (layer "F.Cu") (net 30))
 (segment (start 134.75 90.8495) (end 134.5005 90.6) (width 0.3) (layer "F.Cu") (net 30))
 (segment (start 137.82 90.58) (end 137.8 90.6) (width 0.3) (layer "F.Cu") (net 30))
 (via (at 137.8 90.6) (size 0.8) (drill 0.4) (layers "F.Cu" "B.Cu") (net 30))
 (via (at 134.5005 90.6) (size 0.8) (drill 0.4) (layers "F.Cu" "B.Cu") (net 30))
 (segment (start 134.5005 90.6) (end 137.8 90.6) (width 0.3) (layer "B.Cu") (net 30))
 (segment (start 134.25 93.249022) (end 134.970978 93.97) (width 0.3) (layer "F.Cu") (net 29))
 (segment (start 134.25 92.25) (end 134.25 93.249022) (width 0.3) (layer "F.Cu") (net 29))
 (segment (start 139.35 93.97) (end 140.2 93.12) (width 0.3) (layer "F.Cu") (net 29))
 (segment (start 134.970978 93.97) (end 139.35 93.97) (width 0.3) (layer "F.Cu") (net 29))
 (segment (start 134.60952 95.66) (end 133.74952 94.8) (width 0.3) (layer "F.Cu") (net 28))
 (segment (start 140.2 95.66) (end 134.60952 95.66) (width 0.3) (layer "F.Cu") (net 28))
 (segment (start 133.74952 94.8) (end 133.75 94.79952) (width 0.3) (layer "F.Cu") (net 28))
 (segment (start 133.75 94.79952) (end 133.75 92.25) (width 0.3) (layer "F.Cu") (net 28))
 (segment (start 134.2 98.2) (end 140.2 98.2) (width 0.3) (layer "F.Cu") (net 27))
 (segment (start 133.25 92.25) (end 133.25 97.25) (width 0.3) (layer "F.Cu") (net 27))
 (segment (start 133.25 97.25) (end 134.2 98.2) (width 0.3) (layer "F.Cu") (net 27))
 (segment (start 134.25 71.13) (end 140.2 65.18) (width 0.3) (layer "F.Cu") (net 11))
 (segment (start 134.25 78.55) (end 134.25 71.13) (width 0.3) (layer "F.Cu") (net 11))
 (segment (start 134.75 78.55) (end 134.75 73.17) (width 0.3) (layer "F.Cu") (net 10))
 (segment (start 134.75 73.17) (end 140.2 67.72) (width 0.3) (layer "F.Cu") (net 10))
 (segment (start 135.25 75.21) (end 140.2 70.26) (width 0.3) (layer "F.Cu") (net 9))
 (segment (start 135.25 78.55) (end 135.25 75.21) (width 0.3) (layer "F.Cu") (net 9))
 (segment (start 135.75 78.55) (end 135.75 77.25) (width 0.3) (layer "F.Cu") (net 8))
 (segment (start 135.75 77.25) (end 140.2 72.8) (width 0.3) (layer "F.Cu") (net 8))
 (segment (start 136.25 78.55) (end 136.25 77.550978) (width 0.3) (layer "F.Cu") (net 7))
 (segment (start 138.460978 75.34) (end 140.2 75.34) (width 0.3) (layer "F.Cu") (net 7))
 (segment (start 136.25 77.550978) (end 138.460978 75.34) (width 0.3) (layer "F.Cu") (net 7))
 (segment (start 136.75 78.55) (end 139.53 78.55) (width 0.3) (layer "F.Cu") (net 6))
 (segment (start 139.53 78.55) (end 140.2 77.88) (width 0.3) (layer "F.Cu") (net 6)))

